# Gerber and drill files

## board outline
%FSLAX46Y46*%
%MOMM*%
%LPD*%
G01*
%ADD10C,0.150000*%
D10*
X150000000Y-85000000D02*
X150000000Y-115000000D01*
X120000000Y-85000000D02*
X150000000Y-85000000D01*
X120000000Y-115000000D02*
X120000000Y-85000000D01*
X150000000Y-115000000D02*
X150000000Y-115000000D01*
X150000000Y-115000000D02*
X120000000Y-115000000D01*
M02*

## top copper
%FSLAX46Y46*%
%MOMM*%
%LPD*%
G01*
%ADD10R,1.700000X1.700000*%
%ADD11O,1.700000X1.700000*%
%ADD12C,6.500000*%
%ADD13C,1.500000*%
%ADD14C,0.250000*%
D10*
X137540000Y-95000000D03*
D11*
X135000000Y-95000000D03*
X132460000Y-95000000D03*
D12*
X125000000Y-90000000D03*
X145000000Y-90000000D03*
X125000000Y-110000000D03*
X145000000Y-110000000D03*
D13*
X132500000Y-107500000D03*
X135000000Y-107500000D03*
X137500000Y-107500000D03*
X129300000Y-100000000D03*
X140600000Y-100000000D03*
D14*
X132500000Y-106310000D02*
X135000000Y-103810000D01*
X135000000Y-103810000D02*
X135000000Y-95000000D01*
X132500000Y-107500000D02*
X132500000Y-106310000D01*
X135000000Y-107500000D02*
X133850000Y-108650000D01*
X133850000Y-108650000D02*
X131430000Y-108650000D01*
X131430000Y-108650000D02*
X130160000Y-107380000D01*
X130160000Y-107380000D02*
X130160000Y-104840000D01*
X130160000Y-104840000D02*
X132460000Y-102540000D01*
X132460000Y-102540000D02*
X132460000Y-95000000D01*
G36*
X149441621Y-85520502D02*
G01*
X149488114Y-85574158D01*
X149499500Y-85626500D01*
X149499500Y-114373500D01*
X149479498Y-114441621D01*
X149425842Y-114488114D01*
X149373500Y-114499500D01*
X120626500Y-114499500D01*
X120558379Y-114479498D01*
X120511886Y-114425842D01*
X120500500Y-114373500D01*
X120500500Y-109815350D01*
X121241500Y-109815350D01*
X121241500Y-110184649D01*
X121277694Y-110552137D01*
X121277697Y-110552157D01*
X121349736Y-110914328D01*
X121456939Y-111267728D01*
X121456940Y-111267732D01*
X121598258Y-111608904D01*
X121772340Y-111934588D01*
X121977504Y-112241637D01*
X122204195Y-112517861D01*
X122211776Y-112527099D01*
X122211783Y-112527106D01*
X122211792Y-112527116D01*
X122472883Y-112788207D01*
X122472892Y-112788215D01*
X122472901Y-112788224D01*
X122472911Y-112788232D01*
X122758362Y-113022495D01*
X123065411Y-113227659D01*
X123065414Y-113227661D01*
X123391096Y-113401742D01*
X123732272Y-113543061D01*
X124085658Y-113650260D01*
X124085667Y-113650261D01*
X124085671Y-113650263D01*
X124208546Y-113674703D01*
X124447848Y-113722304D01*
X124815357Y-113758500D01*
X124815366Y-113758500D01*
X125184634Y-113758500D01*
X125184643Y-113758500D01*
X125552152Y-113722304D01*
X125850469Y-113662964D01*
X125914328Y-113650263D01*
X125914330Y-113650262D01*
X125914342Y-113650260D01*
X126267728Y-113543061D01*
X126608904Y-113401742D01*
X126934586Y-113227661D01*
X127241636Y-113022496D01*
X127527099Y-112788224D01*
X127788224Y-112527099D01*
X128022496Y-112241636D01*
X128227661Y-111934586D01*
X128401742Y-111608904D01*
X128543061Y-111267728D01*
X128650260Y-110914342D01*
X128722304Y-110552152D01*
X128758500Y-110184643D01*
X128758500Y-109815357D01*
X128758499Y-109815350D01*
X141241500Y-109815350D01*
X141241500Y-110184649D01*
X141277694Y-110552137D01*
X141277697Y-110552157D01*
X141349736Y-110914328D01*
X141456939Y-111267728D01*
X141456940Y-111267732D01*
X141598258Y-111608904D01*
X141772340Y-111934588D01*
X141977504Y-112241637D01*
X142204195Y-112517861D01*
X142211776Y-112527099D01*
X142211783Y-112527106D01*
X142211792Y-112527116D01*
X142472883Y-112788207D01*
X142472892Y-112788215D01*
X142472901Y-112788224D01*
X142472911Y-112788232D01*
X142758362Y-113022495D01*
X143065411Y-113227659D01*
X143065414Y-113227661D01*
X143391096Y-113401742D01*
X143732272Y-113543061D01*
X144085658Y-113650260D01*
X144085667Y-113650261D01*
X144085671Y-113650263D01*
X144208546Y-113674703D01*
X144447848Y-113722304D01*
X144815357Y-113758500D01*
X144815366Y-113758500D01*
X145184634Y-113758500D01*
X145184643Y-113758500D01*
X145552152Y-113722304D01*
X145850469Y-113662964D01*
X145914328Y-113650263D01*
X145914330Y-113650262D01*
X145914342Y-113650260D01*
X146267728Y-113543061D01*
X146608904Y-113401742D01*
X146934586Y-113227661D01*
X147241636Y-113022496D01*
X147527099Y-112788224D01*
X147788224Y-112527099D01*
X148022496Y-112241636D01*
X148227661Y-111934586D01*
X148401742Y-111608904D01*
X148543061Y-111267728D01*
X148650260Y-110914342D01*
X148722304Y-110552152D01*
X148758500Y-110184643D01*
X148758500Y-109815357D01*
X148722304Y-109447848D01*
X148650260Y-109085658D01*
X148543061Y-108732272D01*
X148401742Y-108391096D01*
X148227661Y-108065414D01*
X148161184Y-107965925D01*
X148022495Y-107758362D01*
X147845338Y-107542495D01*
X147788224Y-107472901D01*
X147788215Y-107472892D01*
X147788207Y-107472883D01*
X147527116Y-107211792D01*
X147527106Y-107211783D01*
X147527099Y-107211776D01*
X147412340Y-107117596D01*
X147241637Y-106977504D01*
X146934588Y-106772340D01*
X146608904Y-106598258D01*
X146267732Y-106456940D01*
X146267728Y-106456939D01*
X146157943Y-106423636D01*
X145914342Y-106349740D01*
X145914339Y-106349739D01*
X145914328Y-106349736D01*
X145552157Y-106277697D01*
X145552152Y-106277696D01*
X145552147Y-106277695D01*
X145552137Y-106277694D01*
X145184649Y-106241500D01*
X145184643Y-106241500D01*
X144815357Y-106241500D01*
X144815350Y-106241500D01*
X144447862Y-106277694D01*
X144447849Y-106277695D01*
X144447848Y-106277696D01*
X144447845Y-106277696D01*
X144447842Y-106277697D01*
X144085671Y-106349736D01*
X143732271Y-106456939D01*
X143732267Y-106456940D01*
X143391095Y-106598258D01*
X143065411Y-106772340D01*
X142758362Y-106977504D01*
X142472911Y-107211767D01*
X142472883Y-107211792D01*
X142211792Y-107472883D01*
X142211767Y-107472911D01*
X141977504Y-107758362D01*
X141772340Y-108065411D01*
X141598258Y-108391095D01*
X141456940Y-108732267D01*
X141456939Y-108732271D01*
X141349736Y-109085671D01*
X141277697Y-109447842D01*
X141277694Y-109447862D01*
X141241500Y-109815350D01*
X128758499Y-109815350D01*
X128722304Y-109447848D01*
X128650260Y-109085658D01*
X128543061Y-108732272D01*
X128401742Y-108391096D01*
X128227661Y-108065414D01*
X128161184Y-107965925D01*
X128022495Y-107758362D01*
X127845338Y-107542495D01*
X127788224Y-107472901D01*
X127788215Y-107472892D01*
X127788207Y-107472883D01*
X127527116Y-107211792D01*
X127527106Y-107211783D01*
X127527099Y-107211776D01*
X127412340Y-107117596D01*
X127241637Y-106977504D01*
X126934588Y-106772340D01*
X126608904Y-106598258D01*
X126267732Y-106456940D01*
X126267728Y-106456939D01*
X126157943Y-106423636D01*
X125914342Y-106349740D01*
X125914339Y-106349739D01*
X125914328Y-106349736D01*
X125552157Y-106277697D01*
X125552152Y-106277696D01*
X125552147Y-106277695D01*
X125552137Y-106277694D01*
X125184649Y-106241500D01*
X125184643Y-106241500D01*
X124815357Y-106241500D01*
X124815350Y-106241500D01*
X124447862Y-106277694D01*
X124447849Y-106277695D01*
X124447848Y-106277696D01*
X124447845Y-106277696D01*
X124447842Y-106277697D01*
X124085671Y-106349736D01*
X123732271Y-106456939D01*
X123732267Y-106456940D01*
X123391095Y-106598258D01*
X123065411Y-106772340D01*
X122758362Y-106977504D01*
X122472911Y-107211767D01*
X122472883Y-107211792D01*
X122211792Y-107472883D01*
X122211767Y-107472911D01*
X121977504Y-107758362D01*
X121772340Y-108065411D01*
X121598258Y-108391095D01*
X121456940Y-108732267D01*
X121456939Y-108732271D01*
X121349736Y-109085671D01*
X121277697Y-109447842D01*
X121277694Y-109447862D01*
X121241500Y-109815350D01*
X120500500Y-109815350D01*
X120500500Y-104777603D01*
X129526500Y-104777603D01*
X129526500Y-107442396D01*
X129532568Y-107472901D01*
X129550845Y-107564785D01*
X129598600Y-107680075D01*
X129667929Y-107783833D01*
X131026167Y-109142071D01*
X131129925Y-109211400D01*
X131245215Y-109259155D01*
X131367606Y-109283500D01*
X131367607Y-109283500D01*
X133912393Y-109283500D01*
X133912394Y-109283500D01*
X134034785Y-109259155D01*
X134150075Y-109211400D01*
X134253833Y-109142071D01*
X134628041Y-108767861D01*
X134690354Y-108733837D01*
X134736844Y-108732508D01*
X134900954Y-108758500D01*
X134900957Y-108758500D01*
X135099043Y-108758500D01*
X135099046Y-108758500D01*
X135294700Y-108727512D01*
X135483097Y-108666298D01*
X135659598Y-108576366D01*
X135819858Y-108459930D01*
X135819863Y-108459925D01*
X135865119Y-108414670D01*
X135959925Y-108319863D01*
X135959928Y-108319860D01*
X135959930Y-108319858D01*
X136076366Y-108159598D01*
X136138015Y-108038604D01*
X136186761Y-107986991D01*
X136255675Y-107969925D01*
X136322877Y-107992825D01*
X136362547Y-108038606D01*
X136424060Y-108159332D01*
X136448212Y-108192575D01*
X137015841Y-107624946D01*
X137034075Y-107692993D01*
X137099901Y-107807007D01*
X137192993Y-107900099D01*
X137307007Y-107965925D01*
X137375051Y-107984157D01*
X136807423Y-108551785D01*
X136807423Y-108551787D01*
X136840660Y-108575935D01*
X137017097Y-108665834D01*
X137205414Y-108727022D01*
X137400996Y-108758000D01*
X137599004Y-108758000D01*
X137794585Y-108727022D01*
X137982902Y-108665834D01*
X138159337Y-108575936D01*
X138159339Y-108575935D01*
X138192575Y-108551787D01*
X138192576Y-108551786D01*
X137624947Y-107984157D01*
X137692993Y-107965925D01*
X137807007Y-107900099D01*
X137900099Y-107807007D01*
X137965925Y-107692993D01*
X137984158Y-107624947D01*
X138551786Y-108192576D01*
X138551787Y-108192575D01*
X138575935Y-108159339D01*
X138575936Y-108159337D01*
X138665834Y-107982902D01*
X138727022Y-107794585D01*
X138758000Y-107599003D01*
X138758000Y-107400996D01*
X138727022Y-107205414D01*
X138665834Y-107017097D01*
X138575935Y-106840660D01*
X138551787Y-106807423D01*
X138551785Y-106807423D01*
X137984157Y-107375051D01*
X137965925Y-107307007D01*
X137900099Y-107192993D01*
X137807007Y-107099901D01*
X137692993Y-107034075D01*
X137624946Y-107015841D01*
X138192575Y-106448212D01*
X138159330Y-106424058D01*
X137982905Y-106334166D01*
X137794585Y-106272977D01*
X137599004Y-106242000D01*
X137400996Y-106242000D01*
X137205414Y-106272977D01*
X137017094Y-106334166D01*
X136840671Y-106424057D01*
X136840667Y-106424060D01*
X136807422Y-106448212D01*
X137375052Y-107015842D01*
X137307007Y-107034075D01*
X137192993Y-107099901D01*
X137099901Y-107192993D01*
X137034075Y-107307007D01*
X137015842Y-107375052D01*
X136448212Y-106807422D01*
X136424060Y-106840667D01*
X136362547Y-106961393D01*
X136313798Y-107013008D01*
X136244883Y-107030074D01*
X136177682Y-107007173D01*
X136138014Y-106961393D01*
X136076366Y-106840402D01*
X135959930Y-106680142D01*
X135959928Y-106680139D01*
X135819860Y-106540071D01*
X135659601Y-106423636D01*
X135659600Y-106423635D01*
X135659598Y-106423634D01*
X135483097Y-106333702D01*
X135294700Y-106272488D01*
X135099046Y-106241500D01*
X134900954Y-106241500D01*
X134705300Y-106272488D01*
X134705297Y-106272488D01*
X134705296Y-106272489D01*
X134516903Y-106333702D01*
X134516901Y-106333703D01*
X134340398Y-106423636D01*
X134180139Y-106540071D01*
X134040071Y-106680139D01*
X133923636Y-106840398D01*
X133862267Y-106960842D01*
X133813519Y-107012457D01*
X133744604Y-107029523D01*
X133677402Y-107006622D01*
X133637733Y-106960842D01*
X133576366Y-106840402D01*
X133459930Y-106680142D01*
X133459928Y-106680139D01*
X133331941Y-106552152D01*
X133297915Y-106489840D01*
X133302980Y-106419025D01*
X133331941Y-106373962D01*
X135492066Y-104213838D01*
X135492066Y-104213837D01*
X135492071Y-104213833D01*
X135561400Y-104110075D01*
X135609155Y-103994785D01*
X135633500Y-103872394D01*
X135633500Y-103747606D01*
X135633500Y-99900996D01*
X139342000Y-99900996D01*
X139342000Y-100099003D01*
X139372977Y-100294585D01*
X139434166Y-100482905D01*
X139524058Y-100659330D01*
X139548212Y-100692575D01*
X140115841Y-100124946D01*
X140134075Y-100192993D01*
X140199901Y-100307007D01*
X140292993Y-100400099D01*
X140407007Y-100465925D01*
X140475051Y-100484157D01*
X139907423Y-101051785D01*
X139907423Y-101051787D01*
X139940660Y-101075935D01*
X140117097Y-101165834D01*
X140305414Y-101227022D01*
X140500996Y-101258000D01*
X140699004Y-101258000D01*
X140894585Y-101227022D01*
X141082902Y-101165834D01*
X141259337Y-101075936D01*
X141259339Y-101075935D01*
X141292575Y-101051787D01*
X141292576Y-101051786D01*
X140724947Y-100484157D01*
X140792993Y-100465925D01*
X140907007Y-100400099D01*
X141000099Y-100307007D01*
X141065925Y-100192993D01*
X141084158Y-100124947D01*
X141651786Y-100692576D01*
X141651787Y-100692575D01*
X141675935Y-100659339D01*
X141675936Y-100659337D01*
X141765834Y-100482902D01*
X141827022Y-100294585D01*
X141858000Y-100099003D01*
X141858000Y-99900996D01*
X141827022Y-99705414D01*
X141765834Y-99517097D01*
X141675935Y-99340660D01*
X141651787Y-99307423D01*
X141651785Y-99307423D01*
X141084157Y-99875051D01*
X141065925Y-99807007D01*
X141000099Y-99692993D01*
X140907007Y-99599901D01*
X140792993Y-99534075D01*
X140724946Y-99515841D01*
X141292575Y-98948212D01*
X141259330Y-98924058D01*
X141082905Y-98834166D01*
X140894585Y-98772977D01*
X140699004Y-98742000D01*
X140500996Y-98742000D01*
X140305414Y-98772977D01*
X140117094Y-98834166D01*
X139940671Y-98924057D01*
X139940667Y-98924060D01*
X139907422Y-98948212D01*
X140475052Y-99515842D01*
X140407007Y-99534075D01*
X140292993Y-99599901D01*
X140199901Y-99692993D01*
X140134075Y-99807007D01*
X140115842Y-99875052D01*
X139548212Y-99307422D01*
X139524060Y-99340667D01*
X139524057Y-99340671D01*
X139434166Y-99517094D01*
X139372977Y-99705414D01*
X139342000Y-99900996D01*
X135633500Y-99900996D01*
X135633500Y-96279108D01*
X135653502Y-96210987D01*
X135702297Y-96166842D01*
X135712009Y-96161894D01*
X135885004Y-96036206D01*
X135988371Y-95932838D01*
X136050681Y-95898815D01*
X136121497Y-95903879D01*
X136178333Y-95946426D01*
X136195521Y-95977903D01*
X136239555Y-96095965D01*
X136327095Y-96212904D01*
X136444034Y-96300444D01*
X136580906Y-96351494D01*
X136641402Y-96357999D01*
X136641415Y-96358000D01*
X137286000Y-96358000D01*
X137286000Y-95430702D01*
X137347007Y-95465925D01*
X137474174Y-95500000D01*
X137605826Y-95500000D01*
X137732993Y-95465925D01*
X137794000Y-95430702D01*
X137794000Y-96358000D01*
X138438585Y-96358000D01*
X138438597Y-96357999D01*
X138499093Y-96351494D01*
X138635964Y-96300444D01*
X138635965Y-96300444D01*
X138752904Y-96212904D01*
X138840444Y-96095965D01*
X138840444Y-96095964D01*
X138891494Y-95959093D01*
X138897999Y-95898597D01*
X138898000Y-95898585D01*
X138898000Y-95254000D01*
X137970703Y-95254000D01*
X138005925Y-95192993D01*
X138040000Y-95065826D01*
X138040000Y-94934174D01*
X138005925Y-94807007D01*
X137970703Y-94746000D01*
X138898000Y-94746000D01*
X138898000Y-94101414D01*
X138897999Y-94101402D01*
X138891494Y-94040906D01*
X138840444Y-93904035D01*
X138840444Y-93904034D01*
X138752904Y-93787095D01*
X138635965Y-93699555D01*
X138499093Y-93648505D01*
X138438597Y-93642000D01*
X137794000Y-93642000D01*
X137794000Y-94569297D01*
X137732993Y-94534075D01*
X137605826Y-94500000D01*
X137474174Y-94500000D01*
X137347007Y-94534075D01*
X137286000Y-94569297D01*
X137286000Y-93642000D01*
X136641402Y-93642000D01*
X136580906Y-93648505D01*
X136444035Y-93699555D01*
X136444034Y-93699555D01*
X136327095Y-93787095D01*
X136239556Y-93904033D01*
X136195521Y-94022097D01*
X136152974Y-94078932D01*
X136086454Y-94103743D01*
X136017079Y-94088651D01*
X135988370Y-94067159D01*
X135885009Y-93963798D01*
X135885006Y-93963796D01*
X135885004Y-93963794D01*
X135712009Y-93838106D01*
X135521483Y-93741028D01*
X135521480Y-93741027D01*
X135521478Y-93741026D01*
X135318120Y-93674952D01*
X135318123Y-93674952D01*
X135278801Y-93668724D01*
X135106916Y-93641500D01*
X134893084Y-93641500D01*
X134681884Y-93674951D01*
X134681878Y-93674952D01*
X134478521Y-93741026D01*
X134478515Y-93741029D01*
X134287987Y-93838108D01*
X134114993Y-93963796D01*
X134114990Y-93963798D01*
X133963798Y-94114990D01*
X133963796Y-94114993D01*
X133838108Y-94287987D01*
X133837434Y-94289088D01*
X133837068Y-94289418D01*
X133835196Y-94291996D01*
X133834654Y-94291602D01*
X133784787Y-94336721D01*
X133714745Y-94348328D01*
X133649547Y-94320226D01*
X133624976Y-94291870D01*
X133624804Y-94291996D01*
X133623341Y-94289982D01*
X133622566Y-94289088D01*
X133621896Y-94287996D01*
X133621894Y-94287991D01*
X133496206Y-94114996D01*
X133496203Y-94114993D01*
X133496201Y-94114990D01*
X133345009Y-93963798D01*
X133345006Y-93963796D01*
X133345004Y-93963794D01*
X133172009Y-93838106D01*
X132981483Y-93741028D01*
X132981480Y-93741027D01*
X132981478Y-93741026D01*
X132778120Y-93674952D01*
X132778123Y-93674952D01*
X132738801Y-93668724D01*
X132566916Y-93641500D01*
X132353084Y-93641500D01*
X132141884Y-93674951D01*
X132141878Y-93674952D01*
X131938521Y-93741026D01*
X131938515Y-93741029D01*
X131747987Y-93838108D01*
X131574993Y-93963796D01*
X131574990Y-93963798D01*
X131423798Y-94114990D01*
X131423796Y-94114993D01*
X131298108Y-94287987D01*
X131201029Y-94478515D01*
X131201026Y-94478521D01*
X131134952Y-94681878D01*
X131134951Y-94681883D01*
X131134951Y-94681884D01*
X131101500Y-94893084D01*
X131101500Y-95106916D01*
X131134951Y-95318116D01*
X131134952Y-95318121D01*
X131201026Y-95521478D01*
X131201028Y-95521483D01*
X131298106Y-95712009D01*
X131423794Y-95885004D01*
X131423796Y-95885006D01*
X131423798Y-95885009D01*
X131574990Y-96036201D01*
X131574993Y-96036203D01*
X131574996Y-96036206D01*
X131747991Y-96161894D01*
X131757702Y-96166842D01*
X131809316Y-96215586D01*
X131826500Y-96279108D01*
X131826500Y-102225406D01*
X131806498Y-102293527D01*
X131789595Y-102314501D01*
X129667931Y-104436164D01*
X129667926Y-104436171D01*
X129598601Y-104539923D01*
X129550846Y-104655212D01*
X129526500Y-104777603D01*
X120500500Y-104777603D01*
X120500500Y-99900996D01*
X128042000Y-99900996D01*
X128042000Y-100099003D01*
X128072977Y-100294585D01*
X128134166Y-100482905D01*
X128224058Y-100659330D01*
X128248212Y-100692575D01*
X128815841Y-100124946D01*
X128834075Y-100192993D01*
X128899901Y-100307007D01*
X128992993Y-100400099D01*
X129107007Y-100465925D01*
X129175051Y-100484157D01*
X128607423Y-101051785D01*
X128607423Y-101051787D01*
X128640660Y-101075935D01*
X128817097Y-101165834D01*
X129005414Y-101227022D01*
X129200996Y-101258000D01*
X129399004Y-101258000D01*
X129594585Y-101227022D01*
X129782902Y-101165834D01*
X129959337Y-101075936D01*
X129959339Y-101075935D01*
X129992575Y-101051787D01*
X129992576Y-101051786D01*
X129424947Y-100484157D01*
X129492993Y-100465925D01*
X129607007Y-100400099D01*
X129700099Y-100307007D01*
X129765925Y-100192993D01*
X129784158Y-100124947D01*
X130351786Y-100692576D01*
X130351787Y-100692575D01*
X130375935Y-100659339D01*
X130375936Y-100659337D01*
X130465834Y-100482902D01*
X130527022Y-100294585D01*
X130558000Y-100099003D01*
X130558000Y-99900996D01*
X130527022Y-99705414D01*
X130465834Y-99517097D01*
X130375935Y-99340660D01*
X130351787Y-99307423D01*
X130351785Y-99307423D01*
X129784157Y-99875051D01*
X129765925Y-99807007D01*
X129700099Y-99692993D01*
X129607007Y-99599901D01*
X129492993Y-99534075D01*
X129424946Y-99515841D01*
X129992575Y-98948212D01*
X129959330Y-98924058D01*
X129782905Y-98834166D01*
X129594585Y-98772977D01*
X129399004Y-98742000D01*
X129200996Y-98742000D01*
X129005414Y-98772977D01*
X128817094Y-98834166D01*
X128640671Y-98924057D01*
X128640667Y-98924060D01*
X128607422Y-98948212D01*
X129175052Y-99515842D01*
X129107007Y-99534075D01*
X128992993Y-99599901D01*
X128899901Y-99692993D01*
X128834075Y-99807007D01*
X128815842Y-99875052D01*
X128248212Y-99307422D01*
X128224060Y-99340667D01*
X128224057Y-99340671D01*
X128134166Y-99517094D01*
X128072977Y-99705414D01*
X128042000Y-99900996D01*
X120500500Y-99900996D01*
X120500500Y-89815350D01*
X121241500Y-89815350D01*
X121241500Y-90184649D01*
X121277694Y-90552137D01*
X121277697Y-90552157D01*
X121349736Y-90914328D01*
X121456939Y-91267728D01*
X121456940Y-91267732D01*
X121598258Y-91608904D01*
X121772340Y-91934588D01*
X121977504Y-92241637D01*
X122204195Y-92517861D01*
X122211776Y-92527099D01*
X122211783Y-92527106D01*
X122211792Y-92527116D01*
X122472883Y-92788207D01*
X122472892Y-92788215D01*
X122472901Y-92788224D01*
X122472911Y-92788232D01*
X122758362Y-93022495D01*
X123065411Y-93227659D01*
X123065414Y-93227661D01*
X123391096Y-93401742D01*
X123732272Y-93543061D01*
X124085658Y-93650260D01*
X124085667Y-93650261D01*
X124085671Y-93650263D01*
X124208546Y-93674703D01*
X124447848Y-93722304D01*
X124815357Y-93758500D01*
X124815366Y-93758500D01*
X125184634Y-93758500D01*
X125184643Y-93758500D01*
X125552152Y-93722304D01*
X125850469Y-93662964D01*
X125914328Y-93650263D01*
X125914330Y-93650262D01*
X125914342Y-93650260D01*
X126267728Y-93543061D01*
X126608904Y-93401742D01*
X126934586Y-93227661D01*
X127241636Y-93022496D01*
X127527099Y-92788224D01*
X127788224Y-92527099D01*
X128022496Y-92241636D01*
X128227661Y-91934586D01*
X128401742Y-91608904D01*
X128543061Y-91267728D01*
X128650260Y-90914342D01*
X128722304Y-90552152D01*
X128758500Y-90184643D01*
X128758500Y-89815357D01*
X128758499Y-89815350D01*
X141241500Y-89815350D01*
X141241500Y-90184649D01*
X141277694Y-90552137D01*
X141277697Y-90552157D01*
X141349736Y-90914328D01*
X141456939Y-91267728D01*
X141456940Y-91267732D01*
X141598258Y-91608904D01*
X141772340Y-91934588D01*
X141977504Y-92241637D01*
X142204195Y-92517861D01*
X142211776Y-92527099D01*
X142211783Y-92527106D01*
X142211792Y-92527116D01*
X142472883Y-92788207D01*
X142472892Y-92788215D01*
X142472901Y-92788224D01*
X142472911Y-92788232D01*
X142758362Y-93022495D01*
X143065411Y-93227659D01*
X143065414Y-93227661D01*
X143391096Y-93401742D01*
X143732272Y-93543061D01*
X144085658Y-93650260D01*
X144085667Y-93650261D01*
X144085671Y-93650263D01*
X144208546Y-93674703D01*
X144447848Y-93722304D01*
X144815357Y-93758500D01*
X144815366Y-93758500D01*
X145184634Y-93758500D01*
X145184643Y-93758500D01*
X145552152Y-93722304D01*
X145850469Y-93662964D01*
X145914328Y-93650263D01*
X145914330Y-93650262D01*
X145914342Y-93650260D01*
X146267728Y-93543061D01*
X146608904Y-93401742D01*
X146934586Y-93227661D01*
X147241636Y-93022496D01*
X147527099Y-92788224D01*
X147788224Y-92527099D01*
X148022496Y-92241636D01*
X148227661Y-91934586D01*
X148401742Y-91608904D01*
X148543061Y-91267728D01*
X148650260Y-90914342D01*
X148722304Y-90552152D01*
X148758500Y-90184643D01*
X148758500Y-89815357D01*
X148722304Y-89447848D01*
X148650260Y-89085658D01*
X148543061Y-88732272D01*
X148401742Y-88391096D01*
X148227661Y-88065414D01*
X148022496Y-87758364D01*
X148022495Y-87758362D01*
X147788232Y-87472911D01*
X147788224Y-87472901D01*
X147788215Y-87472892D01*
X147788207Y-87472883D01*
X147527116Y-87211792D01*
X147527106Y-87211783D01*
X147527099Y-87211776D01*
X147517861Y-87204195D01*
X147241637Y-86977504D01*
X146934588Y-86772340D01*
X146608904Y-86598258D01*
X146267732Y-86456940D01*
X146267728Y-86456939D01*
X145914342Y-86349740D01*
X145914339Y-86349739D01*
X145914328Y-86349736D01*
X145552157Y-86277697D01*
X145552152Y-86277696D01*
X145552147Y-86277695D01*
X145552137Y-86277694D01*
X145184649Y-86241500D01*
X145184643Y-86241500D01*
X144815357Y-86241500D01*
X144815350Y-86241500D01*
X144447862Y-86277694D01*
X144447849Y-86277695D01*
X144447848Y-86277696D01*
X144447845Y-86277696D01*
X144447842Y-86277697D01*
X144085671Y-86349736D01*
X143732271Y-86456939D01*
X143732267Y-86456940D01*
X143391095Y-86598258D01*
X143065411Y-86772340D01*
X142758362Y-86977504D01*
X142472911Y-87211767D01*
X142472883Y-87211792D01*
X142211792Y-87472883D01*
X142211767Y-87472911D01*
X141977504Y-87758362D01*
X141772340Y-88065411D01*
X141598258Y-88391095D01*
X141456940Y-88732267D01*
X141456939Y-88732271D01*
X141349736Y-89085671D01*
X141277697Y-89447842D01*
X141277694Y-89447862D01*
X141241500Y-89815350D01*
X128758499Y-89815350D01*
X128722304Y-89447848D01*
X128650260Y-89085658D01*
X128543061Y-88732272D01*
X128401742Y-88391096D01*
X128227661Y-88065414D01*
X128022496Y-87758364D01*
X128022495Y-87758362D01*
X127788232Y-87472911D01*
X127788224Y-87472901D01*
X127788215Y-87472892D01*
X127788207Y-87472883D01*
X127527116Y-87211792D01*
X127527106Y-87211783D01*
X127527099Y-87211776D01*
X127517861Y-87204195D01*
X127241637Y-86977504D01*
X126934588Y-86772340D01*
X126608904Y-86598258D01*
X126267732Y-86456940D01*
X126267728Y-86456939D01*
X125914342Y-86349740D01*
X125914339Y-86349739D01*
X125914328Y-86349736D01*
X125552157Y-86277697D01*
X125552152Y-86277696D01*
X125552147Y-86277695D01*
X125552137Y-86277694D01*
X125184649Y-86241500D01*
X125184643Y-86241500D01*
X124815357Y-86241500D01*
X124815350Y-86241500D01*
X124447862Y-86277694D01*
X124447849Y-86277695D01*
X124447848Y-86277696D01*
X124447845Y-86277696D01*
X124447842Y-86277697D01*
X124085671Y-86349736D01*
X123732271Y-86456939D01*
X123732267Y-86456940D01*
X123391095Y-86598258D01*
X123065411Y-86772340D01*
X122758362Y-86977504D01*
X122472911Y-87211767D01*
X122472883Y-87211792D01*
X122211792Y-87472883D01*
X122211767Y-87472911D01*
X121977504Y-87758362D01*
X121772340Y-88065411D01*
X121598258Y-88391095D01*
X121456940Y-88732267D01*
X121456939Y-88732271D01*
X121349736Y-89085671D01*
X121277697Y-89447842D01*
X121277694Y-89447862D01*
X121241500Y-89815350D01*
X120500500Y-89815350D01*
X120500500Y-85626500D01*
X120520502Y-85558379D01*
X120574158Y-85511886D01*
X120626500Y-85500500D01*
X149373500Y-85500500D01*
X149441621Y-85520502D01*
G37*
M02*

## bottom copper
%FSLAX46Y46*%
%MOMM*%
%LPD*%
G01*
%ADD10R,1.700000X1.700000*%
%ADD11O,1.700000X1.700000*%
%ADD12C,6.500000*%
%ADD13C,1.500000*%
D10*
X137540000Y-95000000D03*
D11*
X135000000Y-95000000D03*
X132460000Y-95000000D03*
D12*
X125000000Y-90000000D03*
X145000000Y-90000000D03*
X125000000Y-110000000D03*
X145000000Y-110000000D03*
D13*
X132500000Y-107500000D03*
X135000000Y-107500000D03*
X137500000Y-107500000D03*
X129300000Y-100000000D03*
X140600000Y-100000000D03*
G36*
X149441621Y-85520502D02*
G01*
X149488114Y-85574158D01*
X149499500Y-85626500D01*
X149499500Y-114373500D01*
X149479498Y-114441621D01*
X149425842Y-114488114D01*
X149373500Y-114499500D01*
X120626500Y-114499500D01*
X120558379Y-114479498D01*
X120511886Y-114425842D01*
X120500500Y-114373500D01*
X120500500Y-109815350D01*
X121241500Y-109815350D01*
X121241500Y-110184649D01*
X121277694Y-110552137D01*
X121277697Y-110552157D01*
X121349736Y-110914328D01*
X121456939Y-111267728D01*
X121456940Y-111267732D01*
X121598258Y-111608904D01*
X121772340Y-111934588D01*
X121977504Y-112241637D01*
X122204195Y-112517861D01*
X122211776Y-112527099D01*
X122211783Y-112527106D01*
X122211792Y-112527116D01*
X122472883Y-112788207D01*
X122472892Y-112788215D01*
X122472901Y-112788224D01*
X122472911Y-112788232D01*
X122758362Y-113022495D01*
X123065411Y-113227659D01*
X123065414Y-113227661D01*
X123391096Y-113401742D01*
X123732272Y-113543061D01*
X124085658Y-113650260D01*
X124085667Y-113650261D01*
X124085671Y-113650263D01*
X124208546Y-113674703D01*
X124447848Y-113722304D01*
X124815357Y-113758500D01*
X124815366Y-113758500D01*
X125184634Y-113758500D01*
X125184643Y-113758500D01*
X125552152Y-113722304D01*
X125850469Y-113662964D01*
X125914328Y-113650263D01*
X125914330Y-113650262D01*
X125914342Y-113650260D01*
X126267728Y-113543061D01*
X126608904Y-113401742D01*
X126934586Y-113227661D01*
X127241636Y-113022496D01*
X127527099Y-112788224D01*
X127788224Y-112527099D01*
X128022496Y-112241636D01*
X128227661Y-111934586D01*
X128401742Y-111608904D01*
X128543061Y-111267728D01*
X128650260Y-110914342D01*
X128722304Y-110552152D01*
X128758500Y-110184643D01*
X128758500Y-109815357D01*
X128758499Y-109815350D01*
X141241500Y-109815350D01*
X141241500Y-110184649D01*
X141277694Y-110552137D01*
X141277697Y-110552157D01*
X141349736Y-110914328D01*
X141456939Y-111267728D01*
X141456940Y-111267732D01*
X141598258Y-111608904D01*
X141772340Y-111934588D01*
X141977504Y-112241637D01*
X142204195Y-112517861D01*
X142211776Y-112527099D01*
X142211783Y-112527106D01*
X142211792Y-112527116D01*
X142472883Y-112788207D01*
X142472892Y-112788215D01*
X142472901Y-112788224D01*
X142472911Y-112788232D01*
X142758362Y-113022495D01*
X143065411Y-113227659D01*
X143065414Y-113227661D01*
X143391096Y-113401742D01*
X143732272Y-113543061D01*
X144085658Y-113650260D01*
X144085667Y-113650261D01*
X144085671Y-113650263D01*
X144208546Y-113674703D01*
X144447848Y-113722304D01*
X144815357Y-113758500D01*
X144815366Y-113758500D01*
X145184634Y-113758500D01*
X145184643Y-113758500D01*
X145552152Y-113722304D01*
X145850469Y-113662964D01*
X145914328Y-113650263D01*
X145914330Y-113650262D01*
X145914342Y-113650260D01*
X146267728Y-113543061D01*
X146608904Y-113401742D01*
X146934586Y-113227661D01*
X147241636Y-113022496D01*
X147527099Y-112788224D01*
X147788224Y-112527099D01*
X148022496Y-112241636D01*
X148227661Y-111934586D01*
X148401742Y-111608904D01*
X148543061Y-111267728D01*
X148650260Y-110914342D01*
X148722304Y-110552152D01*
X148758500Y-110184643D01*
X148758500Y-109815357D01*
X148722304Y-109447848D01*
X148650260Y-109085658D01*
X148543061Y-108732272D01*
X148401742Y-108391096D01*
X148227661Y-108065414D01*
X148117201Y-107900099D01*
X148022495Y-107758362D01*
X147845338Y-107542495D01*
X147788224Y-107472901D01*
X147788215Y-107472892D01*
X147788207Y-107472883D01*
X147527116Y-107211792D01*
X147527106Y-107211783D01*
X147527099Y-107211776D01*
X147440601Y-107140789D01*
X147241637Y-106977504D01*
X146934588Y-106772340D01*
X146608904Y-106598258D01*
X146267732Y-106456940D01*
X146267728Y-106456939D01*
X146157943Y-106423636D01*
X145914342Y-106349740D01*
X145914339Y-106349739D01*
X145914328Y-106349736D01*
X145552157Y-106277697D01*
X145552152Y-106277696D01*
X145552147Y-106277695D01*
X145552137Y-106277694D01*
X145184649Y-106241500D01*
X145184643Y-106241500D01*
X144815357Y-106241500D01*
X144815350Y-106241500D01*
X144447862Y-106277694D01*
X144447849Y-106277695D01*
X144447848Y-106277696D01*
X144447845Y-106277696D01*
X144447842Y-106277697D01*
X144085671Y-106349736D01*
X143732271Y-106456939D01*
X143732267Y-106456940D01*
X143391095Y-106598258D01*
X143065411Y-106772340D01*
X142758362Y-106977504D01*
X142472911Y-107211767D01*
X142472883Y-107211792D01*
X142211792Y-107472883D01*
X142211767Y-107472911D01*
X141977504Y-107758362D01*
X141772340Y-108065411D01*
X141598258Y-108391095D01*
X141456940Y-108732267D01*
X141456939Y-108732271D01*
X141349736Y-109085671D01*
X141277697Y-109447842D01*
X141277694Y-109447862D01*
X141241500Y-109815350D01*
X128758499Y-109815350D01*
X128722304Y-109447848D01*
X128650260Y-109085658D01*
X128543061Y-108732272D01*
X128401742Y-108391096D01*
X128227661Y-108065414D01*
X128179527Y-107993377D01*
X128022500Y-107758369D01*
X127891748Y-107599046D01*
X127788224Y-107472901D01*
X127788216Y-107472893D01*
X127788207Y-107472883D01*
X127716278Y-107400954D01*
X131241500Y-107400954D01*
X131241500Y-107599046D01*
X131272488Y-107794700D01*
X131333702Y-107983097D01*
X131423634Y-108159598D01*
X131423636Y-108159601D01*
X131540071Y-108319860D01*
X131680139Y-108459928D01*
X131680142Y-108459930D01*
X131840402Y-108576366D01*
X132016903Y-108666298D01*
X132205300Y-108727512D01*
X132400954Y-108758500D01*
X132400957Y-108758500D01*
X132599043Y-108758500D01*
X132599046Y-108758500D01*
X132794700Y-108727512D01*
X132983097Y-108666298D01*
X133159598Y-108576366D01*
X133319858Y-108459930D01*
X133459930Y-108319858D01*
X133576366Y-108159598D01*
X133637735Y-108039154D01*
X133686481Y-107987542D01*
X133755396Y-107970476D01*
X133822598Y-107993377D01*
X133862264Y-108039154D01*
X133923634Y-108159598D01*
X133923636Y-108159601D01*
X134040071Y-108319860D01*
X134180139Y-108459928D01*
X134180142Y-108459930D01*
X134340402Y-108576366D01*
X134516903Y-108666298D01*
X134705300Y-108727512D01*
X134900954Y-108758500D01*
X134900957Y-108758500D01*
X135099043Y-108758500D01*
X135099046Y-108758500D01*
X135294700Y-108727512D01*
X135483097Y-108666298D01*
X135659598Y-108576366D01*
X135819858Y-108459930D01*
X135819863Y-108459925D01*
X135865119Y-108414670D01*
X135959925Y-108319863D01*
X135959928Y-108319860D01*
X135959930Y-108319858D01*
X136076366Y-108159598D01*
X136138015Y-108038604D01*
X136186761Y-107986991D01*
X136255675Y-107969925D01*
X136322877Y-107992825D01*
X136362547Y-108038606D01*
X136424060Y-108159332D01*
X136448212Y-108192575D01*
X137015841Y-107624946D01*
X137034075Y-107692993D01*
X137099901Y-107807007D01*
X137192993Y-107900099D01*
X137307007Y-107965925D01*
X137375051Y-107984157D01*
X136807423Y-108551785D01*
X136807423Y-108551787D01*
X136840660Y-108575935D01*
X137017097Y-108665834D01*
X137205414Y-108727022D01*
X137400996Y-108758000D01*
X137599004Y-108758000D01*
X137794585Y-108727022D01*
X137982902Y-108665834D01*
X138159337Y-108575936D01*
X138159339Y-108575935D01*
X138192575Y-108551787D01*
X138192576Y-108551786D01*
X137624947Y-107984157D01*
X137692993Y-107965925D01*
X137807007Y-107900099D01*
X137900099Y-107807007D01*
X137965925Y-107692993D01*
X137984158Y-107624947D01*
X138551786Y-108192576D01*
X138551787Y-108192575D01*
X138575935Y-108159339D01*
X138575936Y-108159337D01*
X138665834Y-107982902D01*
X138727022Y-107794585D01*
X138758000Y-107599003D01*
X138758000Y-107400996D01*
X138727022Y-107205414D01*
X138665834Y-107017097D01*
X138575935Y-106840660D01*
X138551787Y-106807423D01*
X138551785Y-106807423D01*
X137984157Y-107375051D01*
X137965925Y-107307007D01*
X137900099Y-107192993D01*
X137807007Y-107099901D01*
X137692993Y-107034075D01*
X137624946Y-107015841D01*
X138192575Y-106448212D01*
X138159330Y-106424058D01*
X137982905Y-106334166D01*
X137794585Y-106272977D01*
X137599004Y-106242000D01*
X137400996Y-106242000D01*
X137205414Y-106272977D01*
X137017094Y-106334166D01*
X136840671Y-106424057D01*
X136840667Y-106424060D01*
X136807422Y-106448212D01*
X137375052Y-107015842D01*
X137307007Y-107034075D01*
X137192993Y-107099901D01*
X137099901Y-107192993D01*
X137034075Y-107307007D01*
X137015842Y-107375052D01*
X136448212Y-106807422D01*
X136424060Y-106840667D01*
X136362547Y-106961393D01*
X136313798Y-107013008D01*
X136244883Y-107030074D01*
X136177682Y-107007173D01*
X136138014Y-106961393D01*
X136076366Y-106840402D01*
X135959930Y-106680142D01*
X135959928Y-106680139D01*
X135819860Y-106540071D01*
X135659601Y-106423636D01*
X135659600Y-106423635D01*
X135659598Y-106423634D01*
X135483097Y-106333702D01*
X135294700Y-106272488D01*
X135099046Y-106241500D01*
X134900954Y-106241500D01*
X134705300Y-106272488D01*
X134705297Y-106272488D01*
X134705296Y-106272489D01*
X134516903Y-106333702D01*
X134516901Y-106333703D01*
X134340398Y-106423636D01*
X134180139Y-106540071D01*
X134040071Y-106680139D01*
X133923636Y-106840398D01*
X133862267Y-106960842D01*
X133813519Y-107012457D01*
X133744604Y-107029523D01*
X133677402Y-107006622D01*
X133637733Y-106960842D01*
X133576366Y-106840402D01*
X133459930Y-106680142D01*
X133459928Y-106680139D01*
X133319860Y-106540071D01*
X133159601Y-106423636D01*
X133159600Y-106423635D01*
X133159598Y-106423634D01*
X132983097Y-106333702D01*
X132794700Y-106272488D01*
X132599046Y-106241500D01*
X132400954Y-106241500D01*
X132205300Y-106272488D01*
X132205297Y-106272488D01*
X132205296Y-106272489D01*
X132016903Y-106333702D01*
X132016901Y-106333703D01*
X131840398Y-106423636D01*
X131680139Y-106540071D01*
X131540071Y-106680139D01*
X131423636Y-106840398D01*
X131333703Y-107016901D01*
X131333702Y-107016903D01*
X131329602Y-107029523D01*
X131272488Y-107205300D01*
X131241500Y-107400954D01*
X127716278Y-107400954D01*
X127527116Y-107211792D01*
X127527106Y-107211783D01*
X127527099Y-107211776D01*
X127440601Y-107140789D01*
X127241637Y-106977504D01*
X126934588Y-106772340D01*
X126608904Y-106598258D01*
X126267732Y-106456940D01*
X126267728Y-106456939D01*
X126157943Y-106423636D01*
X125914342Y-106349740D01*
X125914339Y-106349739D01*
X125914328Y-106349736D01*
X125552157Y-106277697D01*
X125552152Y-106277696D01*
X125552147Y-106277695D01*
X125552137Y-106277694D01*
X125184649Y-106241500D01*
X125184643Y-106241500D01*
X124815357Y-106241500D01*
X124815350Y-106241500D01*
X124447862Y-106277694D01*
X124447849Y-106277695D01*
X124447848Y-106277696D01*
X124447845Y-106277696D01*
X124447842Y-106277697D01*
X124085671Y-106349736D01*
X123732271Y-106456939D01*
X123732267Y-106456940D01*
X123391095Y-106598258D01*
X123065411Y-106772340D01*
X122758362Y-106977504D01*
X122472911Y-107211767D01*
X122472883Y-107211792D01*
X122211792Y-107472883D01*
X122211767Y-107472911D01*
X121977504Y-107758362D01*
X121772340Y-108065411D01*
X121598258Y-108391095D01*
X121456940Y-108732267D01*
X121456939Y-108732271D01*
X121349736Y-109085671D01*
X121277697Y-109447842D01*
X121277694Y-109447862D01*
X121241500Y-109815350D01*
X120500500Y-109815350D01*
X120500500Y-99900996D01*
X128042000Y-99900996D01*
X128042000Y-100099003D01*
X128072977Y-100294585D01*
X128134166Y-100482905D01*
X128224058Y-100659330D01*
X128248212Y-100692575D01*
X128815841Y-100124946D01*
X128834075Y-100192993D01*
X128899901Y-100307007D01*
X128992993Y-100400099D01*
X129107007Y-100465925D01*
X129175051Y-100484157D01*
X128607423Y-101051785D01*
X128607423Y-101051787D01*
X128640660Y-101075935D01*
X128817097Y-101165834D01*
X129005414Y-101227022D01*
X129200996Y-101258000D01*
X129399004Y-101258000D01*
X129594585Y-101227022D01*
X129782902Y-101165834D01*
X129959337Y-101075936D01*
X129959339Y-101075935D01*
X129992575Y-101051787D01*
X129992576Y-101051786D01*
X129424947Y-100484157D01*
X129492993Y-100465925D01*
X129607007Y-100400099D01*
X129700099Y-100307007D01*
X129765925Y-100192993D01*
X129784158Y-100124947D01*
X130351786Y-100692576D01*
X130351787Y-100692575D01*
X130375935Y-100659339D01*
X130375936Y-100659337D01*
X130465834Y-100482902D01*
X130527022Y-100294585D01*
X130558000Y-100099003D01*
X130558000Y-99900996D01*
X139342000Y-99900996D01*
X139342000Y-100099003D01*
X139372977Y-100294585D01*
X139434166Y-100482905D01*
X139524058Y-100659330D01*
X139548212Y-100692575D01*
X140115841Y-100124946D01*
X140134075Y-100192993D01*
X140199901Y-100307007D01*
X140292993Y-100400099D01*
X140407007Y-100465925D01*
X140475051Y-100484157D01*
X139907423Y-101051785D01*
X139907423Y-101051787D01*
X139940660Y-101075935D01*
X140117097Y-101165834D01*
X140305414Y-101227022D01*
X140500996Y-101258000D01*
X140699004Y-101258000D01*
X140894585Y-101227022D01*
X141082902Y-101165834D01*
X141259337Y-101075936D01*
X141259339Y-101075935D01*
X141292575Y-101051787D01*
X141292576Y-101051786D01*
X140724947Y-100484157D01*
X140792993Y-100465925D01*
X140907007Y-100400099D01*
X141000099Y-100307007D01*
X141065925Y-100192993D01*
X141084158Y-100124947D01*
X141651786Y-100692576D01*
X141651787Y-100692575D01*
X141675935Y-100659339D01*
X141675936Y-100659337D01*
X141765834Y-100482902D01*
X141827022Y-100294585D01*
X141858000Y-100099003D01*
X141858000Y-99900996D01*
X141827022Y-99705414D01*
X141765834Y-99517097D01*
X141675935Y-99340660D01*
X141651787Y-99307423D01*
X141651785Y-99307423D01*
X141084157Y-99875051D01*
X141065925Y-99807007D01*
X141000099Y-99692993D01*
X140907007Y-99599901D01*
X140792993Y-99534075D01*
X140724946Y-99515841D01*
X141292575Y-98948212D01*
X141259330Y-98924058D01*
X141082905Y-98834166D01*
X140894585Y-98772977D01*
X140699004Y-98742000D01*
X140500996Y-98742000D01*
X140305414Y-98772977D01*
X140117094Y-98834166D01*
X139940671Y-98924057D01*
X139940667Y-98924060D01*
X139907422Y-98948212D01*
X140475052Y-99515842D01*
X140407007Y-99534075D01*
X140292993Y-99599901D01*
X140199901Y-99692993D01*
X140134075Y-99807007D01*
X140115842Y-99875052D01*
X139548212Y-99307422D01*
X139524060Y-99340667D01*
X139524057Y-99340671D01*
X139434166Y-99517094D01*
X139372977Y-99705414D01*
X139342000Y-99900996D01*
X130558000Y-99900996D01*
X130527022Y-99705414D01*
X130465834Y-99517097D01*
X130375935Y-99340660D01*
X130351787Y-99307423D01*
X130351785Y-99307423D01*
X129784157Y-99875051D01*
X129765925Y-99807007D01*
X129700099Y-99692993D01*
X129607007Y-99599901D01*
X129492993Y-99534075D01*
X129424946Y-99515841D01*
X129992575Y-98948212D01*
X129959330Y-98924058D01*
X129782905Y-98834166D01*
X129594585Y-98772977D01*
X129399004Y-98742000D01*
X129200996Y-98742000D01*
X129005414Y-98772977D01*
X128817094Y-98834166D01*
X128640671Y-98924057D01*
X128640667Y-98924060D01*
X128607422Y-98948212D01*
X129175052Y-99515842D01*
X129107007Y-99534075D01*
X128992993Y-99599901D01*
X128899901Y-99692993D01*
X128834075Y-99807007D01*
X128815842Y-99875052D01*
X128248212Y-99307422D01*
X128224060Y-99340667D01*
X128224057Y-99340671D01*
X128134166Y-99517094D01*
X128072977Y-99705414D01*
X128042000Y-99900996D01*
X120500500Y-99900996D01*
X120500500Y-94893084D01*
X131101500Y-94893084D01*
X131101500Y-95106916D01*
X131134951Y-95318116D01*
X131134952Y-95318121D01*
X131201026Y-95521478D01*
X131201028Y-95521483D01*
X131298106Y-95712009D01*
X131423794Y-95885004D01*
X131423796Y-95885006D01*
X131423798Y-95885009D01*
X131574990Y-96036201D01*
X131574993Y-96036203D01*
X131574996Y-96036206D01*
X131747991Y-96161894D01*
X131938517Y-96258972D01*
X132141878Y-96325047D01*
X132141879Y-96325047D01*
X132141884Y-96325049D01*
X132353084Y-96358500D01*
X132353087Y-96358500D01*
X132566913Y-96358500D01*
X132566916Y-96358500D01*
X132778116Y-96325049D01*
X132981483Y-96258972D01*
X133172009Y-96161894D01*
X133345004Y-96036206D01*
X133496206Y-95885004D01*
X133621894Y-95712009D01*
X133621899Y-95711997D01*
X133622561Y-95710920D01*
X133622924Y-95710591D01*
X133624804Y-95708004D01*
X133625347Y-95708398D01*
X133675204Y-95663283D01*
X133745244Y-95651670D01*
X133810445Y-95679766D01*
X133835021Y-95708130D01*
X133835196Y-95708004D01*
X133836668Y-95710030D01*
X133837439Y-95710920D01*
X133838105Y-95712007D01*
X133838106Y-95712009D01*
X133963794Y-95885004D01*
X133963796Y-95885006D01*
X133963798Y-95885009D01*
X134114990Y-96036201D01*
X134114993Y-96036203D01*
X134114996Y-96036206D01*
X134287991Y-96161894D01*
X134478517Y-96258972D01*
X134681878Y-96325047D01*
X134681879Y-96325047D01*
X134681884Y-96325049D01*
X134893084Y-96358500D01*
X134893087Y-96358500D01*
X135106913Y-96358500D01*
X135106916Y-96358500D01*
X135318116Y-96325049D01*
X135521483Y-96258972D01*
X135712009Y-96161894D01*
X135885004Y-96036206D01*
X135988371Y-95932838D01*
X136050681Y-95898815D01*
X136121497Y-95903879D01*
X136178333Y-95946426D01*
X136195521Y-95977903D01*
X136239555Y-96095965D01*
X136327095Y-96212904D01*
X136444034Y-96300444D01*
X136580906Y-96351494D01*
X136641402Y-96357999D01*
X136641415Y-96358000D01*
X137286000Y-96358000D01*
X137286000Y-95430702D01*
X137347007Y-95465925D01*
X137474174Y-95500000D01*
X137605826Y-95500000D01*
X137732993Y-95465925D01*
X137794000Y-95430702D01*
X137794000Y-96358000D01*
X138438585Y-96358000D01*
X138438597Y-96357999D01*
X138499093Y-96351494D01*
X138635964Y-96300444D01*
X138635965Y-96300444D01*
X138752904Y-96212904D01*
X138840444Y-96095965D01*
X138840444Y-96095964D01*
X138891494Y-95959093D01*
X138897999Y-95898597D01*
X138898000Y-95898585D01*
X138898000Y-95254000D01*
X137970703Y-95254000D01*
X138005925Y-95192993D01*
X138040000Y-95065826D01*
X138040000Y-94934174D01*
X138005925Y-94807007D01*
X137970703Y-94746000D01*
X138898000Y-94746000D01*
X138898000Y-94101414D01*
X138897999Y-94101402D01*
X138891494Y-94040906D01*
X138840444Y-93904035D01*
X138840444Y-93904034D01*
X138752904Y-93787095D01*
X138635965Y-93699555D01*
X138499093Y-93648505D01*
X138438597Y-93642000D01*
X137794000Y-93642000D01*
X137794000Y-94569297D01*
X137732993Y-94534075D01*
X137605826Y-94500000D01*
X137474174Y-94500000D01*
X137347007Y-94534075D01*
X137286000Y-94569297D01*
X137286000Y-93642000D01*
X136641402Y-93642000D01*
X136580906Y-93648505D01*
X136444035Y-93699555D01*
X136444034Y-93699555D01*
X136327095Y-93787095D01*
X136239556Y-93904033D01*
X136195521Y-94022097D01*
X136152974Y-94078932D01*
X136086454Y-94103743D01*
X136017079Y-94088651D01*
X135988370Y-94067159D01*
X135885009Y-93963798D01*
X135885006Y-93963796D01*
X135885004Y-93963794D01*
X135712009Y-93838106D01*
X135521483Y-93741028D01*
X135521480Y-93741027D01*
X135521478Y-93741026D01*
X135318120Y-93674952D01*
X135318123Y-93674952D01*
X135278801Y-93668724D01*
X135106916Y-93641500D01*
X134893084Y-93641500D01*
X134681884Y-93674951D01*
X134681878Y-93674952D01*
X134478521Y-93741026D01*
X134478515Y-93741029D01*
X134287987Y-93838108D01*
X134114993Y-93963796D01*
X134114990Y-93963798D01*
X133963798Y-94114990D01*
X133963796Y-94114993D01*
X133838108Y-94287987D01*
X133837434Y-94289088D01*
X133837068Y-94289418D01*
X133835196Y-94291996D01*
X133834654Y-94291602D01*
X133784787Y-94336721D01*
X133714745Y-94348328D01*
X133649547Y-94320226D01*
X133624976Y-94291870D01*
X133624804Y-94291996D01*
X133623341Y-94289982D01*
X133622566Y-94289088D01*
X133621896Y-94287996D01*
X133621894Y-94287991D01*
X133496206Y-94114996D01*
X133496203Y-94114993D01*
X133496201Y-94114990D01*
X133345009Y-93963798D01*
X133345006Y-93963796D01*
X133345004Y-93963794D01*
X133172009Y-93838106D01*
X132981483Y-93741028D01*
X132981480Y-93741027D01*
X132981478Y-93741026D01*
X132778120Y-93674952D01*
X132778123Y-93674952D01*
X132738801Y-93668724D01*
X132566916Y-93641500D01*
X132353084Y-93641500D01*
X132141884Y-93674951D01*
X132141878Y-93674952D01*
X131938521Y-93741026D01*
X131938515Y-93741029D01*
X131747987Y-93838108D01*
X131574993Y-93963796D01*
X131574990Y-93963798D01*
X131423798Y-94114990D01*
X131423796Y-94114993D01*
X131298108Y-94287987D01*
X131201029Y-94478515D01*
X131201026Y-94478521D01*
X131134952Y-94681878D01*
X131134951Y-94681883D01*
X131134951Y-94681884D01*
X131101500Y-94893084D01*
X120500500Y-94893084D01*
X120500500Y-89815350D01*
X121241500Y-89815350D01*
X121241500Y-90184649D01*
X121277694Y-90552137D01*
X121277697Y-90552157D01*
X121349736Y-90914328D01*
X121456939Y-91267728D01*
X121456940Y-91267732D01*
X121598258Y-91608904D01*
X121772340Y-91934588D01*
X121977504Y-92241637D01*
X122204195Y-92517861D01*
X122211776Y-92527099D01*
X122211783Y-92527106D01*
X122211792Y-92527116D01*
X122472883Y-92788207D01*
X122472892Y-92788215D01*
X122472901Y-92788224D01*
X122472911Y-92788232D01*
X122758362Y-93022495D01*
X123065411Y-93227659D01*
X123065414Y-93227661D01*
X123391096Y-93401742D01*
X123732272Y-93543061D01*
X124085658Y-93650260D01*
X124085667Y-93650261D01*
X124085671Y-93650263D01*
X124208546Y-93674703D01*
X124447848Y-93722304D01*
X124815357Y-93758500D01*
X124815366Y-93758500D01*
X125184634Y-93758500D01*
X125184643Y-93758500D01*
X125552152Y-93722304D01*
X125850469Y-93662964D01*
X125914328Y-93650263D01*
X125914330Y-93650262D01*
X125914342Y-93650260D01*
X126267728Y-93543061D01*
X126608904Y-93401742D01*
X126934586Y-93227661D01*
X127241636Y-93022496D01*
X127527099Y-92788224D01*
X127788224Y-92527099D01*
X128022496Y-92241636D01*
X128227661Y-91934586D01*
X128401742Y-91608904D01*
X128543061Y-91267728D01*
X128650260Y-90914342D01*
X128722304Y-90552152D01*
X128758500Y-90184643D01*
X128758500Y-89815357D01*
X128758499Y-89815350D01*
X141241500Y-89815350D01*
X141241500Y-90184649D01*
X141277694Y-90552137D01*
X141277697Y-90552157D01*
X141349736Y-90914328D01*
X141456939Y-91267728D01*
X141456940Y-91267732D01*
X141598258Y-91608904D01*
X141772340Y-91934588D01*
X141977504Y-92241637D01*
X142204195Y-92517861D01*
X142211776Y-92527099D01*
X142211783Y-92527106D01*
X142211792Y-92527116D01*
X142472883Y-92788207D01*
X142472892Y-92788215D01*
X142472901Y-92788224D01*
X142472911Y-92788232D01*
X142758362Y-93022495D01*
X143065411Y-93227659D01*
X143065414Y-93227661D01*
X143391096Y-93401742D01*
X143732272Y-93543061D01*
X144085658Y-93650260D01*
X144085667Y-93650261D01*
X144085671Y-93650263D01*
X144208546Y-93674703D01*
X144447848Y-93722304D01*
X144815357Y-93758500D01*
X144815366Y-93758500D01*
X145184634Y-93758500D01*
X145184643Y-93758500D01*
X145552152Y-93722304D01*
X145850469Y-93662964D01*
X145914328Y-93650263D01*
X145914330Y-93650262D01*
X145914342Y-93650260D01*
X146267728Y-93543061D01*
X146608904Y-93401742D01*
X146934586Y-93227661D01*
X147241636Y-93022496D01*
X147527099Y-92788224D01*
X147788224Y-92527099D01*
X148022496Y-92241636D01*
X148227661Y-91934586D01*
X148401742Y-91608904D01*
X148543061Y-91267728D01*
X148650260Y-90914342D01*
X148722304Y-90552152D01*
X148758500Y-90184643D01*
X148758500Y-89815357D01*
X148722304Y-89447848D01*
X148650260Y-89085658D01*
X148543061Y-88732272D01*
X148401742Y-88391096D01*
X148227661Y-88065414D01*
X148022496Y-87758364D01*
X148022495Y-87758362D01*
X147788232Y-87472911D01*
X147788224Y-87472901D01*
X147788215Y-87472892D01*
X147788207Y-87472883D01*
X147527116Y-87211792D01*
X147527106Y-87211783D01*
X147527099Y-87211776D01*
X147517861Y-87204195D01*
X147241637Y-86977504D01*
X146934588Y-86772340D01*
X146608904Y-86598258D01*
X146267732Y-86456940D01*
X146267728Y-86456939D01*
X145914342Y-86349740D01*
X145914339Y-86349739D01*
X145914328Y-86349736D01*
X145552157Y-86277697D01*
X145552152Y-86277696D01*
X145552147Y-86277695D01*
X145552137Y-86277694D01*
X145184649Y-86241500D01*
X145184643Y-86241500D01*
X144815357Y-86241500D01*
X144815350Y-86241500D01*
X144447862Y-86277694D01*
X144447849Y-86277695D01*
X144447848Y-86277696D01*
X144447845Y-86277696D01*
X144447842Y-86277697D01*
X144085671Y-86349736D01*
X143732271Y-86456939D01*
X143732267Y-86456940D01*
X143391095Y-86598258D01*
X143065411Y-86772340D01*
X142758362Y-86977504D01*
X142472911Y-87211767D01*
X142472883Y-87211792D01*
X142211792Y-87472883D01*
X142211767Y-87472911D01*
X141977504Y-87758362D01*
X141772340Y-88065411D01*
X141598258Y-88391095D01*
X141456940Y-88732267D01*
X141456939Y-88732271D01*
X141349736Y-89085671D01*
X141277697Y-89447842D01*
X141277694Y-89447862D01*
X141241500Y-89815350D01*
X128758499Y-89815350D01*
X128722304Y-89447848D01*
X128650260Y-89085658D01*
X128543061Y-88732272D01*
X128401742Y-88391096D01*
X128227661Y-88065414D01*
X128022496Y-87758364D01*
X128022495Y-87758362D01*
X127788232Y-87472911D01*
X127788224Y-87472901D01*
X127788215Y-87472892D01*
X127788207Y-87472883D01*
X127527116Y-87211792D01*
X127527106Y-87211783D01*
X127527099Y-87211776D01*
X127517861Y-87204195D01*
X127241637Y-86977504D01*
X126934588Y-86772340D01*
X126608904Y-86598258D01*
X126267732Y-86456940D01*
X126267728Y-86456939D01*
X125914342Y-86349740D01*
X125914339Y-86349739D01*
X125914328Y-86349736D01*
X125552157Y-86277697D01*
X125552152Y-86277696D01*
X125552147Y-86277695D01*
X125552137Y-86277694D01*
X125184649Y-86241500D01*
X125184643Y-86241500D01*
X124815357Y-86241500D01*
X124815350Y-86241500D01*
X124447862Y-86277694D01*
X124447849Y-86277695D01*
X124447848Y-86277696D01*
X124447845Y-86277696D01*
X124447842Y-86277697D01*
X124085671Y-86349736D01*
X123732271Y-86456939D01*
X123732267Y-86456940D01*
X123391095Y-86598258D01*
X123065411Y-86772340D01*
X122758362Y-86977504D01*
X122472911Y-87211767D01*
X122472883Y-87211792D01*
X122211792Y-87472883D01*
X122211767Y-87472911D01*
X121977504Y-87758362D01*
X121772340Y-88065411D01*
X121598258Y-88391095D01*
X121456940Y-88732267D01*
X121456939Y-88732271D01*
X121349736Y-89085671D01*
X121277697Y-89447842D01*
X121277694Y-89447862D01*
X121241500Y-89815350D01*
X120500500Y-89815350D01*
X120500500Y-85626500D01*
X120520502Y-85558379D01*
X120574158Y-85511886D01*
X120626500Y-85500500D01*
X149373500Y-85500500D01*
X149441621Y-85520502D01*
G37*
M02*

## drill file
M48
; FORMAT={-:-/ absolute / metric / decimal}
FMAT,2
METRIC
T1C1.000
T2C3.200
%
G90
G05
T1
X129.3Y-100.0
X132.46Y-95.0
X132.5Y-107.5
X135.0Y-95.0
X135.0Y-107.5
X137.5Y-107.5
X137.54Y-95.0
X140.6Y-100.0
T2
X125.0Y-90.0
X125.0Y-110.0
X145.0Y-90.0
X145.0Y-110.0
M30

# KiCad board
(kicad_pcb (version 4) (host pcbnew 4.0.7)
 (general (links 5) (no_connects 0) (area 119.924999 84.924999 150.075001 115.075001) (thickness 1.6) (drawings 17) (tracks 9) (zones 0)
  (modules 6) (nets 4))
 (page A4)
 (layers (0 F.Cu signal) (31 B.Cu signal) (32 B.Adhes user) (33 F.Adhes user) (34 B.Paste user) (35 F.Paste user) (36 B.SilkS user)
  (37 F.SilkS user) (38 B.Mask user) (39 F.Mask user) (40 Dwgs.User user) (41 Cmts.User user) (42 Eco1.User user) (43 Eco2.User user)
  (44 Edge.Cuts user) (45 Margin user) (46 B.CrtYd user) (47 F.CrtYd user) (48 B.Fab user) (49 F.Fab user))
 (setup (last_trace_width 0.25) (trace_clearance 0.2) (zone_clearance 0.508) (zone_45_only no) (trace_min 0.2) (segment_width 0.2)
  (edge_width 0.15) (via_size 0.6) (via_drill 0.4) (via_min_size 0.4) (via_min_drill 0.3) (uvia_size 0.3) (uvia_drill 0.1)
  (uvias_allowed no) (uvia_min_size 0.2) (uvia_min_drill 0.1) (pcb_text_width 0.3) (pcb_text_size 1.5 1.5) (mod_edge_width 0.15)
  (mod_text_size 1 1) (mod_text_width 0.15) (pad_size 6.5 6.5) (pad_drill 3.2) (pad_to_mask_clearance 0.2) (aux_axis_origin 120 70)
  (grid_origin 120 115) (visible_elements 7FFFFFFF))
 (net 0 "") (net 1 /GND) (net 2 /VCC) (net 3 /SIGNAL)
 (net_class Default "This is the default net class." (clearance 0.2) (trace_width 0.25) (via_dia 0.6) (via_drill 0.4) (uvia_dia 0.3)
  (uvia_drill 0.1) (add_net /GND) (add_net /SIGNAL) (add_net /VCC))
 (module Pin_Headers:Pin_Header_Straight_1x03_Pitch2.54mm (layer B.Cu) (at 137.54 95 90)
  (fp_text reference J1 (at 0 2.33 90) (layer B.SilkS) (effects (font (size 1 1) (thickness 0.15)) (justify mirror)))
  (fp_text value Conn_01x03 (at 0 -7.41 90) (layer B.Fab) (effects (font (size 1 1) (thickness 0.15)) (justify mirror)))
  (pad 1 thru_hole rect (at 0 0 90) (size 1.7 1.7) (drill 1) (layers *.Cu *.Mask) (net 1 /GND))
  (pad 2 thru_hole oval (at 0 -2.54 90) (size 1.7 1.7) (drill 1) (layers *.Cu *.Mask) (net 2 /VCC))
  (pad 3 thru_hole oval (at 0 -5.08 90) (size 1.7 1.7) (drill 1) (layers *.Cu *.Mask) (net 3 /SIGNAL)))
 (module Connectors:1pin (layer F.Cu) (at 125 90)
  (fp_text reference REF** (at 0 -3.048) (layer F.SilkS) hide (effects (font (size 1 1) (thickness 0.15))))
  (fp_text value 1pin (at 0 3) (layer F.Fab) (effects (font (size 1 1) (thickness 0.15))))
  (pad ~ thru_hole circle (at 0 0) (size 6.5 6.5) (drill 3.2) (layers *.Cu *.Mask)))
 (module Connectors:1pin (layer F.Cu) (at 145 90)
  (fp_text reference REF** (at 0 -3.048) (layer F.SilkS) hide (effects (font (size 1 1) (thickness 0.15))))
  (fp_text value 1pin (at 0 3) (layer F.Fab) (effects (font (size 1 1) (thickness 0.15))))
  (pad ~ thru_hole circle (at 0 0) (size 6.5 6.5) (drill 3.2) (layers *.Cu *.Mask)))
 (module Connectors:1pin (layer F.Cu) (at 125 110)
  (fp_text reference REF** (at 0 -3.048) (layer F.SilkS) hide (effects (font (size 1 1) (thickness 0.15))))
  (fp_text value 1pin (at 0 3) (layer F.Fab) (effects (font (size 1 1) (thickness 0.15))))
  (pad ~ thru_hole circle (at 0 0) (size 6.5 6.5) (drill 3.2) (layers *.Cu *.Mask)))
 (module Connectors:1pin (layer F.Cu) (at 145 110)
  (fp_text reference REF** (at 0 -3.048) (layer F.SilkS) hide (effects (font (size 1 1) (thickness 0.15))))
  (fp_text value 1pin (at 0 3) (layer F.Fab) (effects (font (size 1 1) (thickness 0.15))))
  (pad ~ thru_hole circle (at 0 0) (size 6.5 6.5) (drill 3.2) (layers *.Cu *.Mask)))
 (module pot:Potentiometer (layer F.Cu) (at 135 100)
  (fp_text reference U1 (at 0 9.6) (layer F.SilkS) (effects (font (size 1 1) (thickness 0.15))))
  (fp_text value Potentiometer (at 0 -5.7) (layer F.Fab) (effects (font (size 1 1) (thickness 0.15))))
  (pad 1 thru_hole circle (at -2.5 7.5) (size 1.5 1.5) (drill 1) (layers *.Cu *.Mask) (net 2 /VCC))
  (pad 2 thru_hole circle (at 0 7.5) (size 1.5 1.5) (drill 1) (layers *.Cu *.Mask) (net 3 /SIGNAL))
  (pad 3 thru_hole circle (at 2.5 7.5) (size 1.5 1.5) (drill 1) (layers *.Cu *.Mask) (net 1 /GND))
  (pad 4 thru_hole circle (at -5.7 0) (size 1.5 1.5) (drill 1) (layers *.Cu *.Mask) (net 1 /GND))
  (pad 5 thru_hole circle (at 5.6 0) (size 1.5 1.5) (drill 1) (layers *.Cu *.Mask) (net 1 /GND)))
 (gr_line (start 150 85) (end 150 115) (layer Edge.Cuts) (width 0.15))
 (gr_line (start 120 85) (end 150 85) (layer Edge.Cuts) (width 0.15))
 (gr_line (start 120 115) (end 120 85) (layer Edge.Cuts) (width 0.15))
 (gr_line (start 150 115) (end 150 115) (layer Edge.Cuts) (width 0.15))
 (gr_line (start 150 115) (end 120 115) (layer Edge.Cuts) (width 0.15))
 (segment (start 132.5 106.31) (end 135 103.81) (width 0.25) (layer F.Cu) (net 2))
 (segment (start 135 103.81) (end 135 95) (width 0.25) (layer F.Cu) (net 2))
 (segment (start 132.5 107.5) (end 132.5 106.31) (width 0.25) (layer F.Cu) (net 2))
 (segment (start 135 107.5) (end 133.85 108.65) (width 0.25) (layer F.Cu) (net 3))
 (segment (start 133.85 108.65) (end 131.43 108.65) (width 0.25) (layer F.Cu) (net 3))
 (segment (start 131.43 108.65) (end 130.16 107.38) (width 0.25) (layer F.Cu) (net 3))
 (segment (start 130.16 107.38) (end 130.16 104.84) (width 0.25) (layer F.Cu) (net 3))
 (segment (start 130.16 104.84) (end 132.46 102.54) (width 0.25) (layer F.Cu) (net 3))
 (segment (start 132.46 102.54) (end 132.46 95) (width 0.25) (layer F.Cu) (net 3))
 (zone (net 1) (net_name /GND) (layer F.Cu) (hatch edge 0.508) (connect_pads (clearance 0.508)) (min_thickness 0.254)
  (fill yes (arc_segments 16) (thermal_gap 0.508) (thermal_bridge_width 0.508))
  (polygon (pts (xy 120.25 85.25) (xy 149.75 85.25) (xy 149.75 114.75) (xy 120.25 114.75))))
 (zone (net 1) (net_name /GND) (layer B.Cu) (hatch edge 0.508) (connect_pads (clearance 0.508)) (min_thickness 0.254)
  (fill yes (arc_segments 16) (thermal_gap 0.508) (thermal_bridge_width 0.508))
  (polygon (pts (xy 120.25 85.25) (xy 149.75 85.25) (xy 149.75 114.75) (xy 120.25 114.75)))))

